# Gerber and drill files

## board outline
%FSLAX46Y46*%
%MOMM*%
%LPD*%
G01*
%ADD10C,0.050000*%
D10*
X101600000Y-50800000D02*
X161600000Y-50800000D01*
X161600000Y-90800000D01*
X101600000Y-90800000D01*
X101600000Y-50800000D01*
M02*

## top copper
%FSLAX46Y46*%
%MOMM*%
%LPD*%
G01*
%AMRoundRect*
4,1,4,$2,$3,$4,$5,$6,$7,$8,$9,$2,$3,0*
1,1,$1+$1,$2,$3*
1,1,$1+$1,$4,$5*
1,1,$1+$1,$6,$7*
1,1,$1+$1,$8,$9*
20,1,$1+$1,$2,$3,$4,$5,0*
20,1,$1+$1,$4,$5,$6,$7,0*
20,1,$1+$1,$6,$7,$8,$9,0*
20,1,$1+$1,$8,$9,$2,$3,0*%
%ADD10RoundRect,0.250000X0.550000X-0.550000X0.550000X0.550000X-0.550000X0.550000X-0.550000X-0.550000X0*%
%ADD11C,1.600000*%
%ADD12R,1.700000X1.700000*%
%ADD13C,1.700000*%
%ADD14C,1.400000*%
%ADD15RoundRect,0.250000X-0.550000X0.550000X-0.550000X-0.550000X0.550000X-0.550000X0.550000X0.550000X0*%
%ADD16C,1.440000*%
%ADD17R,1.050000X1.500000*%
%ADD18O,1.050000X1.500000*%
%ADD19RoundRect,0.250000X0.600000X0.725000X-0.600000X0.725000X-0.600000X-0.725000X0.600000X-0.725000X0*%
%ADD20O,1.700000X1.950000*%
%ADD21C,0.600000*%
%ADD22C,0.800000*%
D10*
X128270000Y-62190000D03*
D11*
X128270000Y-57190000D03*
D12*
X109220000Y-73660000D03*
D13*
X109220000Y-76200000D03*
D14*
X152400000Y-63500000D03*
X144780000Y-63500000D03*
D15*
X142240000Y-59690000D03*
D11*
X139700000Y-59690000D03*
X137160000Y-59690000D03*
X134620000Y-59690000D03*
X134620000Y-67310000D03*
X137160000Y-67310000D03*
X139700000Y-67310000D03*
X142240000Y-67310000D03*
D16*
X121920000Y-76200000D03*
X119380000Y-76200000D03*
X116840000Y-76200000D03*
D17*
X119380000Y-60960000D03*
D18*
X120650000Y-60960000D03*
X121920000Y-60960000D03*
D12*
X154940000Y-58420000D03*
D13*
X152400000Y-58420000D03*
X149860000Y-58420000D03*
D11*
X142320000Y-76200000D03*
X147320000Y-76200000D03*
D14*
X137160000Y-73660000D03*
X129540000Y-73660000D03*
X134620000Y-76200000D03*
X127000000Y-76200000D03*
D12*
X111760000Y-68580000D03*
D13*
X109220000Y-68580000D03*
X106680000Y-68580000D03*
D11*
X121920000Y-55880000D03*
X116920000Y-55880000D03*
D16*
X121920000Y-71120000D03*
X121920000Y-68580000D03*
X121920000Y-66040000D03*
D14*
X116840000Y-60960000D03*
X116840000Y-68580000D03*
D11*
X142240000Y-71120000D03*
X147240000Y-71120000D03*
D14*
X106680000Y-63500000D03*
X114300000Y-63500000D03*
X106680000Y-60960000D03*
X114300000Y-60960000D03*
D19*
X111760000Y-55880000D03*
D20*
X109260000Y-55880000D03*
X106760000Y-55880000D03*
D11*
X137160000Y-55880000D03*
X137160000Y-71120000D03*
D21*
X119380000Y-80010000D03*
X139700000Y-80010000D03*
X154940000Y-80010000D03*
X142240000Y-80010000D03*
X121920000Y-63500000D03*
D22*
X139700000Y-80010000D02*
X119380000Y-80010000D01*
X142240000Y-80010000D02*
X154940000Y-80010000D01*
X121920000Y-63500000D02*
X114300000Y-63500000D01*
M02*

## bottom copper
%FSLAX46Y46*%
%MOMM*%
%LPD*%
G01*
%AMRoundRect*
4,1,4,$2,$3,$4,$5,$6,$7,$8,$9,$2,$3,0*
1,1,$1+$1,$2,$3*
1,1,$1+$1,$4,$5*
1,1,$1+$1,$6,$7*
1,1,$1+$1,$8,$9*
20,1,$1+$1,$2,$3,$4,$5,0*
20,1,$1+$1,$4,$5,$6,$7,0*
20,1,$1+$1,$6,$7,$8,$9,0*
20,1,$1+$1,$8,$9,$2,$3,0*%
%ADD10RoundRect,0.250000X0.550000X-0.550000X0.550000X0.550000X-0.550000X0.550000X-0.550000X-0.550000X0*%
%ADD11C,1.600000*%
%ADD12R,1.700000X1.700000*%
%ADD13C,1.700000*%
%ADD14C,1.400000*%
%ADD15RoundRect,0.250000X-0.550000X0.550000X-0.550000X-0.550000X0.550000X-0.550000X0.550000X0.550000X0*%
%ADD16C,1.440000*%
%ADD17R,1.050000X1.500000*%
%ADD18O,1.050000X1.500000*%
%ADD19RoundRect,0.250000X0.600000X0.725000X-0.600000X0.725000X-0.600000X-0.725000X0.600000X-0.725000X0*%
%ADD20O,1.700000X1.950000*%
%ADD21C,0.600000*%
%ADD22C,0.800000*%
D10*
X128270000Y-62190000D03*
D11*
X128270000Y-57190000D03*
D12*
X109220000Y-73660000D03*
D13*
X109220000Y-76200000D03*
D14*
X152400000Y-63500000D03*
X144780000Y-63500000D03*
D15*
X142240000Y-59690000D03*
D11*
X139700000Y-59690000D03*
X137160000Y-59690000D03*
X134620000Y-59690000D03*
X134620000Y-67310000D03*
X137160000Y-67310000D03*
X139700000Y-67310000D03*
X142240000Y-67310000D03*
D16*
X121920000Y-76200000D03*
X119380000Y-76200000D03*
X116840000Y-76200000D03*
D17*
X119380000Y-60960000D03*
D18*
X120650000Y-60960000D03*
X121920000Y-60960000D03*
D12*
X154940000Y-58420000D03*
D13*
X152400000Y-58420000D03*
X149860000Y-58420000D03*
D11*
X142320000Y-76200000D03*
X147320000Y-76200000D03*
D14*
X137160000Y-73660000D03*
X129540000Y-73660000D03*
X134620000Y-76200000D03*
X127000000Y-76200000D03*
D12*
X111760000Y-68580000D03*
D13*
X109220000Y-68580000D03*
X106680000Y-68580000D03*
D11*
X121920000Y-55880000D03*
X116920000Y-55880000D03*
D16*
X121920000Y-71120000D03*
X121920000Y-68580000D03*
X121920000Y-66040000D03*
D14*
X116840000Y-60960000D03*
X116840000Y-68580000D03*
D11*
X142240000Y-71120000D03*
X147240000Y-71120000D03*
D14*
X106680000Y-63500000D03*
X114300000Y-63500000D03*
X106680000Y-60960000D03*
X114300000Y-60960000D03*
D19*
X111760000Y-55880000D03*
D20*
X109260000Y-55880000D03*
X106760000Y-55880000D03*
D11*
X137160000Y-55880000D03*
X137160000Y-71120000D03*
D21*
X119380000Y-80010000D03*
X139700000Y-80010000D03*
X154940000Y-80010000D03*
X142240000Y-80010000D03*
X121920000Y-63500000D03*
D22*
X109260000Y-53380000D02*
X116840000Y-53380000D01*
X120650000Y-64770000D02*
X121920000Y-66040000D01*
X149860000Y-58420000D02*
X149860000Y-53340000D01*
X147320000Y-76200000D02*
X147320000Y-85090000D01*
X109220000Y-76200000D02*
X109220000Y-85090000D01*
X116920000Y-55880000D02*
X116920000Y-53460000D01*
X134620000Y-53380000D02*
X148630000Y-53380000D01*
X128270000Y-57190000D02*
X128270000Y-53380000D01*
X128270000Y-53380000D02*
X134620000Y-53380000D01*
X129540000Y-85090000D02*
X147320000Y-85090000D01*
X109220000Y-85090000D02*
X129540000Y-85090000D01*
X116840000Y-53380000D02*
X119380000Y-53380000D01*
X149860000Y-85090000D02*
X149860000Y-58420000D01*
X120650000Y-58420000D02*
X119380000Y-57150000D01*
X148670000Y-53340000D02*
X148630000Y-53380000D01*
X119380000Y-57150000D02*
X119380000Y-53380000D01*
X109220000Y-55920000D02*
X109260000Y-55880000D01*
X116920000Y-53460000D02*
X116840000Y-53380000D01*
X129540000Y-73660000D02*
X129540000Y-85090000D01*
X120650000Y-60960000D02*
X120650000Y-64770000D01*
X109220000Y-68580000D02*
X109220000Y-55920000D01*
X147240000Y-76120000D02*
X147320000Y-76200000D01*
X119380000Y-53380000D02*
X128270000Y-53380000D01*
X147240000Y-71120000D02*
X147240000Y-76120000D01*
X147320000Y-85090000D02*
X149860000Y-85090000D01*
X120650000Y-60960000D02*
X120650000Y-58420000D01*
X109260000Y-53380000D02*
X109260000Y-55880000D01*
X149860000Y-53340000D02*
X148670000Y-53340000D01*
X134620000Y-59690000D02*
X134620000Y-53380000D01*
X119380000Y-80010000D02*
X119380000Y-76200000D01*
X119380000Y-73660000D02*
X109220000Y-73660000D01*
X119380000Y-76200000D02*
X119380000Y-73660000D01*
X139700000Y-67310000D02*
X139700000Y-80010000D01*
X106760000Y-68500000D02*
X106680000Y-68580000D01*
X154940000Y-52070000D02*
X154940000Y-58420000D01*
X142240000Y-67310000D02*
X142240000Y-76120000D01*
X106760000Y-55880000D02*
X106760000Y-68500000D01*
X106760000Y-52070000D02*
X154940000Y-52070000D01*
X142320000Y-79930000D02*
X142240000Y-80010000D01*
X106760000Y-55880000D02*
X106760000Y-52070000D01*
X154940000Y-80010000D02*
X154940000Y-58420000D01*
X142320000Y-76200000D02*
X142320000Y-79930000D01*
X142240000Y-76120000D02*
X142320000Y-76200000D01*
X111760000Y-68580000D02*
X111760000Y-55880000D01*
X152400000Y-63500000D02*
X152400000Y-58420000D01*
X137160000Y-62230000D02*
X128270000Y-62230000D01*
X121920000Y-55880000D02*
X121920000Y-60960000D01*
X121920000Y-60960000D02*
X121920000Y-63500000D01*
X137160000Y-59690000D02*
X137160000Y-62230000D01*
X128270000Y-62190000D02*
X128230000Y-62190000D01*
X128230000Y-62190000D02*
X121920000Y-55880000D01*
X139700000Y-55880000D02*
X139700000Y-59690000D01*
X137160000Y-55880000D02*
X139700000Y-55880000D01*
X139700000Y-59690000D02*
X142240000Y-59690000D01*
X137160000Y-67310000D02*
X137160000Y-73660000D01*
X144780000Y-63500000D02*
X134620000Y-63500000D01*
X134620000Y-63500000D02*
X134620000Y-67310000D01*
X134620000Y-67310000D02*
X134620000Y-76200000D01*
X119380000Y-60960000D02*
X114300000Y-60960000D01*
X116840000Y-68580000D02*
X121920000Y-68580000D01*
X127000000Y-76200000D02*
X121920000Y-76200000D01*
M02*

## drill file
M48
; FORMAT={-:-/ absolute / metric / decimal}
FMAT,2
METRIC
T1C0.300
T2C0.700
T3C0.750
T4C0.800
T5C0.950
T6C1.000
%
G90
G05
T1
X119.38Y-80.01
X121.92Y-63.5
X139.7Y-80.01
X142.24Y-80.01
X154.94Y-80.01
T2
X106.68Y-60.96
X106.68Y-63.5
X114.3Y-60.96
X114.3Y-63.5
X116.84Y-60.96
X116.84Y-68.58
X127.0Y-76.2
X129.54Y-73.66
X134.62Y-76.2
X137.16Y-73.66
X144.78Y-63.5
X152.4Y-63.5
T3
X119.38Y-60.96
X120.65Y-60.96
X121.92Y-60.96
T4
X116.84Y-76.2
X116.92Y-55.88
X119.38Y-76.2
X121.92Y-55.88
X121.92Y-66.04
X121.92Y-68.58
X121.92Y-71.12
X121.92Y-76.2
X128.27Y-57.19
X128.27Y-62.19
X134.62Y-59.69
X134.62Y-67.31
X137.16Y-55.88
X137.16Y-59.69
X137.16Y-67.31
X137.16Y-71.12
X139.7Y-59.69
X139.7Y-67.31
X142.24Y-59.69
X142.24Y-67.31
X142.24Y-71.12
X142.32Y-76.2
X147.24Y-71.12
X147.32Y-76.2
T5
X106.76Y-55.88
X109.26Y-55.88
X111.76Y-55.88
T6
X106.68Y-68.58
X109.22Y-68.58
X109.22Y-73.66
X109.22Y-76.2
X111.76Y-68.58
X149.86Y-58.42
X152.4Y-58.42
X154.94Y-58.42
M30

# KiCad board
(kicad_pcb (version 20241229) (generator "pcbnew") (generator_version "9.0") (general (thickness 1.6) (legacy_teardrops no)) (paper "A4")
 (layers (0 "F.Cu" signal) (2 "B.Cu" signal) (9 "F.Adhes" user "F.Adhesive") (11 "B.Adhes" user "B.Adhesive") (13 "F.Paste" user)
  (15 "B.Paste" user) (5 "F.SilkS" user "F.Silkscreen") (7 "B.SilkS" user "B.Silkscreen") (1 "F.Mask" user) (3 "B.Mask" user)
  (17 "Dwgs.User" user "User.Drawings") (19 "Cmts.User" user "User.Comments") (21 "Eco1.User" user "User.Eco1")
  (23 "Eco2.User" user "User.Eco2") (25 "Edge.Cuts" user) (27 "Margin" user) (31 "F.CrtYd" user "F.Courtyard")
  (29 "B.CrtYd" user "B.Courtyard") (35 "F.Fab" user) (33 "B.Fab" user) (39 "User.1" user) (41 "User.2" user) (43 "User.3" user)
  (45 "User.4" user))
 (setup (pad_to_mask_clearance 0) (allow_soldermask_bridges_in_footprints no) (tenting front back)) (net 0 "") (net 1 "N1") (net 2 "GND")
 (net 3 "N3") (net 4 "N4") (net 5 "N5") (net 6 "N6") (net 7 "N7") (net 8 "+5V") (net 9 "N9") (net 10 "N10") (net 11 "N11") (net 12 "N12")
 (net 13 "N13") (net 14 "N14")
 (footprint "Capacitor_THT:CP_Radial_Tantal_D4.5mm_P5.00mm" (layer "F.Cu") (at 128.27 62.19 90)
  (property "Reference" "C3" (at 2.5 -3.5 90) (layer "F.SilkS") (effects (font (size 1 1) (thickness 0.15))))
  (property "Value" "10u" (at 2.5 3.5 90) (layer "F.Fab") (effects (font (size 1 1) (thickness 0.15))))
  (pad "1" thru_hole roundrect (at 0 0 90) (size 1.6 1.6) (drill 0.8) (layers "*.Cu" "*.Mask") (remove_unused_layers no)
   (roundrect_rratio 0.15625) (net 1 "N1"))
  (pad "2" thru_hole circle (at 5 0 90) (size 1.6 1.6) (drill 0.8) (layers "*.Cu" "*.Mask") (remove_unused_layers no) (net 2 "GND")))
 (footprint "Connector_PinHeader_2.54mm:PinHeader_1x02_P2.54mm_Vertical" (layer "F.Cu") (at 109.22 73.66)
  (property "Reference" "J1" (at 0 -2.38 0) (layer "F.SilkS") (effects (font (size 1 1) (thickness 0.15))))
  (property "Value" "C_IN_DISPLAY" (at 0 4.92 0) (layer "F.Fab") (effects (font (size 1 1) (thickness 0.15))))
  (pad "1" thru_hole rect (at 0 0) (size 1.7 1.7) (drill 1) (layers "*.Cu" "*.Mask") (remove_unused_layers no) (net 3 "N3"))
  (pad "2" thru_hole circle (at 0 2.54) (size 1.7 1.7) (drill 1) (layers "*.Cu" "*.Mask") (remove_unused_layers no) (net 2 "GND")))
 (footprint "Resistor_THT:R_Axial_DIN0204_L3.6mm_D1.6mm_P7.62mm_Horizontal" (layer "F.Cu") (at 152.4 63.5 180)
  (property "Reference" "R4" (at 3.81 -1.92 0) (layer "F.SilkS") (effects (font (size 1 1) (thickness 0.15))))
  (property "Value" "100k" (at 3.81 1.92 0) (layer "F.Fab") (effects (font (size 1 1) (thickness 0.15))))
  (pad "1" thru_hole circle (at 0 0 180) (size 1.4 1.4) (drill 0.7) (layers "*.Cu" "*.Mask") (remove_unused_layers no) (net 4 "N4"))
  (pad "2" thru_hole circle (at 7.62 0 180) (size 1.4 1.4) (drill 0.7) (layers "*.Cu" "*.Mask") (remove_unused_layers no) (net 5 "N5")))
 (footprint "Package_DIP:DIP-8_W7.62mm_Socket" (layer "F.Cu") (at 142.24 59.69 -90)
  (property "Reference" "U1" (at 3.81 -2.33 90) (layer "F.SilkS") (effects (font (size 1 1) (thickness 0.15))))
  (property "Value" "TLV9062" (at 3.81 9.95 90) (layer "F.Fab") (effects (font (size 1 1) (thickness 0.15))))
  (pad "1" thru_hole roundrect (at 0 0 270) (size 1.6 1.6) (drill 0.8) (layers "*.Cu" "*.Mask") (remove_unused_layers no)
   (roundrect_rratio 0.15625) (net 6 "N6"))
  (pad "2" thru_hole circle (at 0 2.54 270) (size 1.6 1.6) (drill 0.8) (layers "*.Cu" "*.Mask") (remove_unused_layers no) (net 6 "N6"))
  (pad "3" thru_hole circle (at 0 5.08 270) (size 1.6 1.6) (drill 0.8) (layers "*.Cu" "*.Mask") (remove_unused_layers no) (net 1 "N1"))
  (pad "4" thru_hole circle (at 0 7.62 270) (size 1.6 1.6) (drill 0.8) (layers "*.Cu" "*.Mask") (remove_unused_layers no) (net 2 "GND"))
  (pad "5" thru_hole circle (at 7.62 7.62 270) (size 1.6 1.6) (drill 0.8) (layers "*.Cu" "*.Mask") (remove_unused_layers no) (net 5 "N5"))
  (pad "6" thru_hole circle (at 7.62 5.08 270) (size 1.6 1.6) (drill 0.8) (layers "*.Cu" "*.Mask") (remove_unused_layers no) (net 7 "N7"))
  (pad "7" thru_hole circle (at 7.62 2.54 270) (size 1.6 1.6) (drill 0.8) (layers "*.Cu" "*.Mask") (remove_unused_layers no) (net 3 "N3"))
  (pad "8" thru_hole circle (at 7.62 0 270) (size 1.6 1.6) (drill 0.8) (layers "*.Cu" "*.Mask") (remove_unused_layers no) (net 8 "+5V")))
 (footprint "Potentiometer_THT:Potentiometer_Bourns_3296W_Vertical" (layer "F.Cu") (at 121.92 76.2)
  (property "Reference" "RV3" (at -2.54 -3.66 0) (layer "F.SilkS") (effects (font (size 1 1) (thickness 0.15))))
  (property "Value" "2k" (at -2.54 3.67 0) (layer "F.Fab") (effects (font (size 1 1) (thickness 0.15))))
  (pad "1" thru_hole circle (at 0 0) (size 1.44 1.44) (drill 0.8) (layers "*.Cu" "*.Mask") (remove_unused_layers no) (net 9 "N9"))
  (pad "2" thru_hole circle (at -2.54 0) (size 1.44 1.44) (drill 0.8) (layers "*.Cu" "*.Mask") (remove_unused_layers no) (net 3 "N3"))
  (pad "3" thru_hole circle (at -5.08 0) (size 1.44 1.44) (drill 0.8) (layers "*.Cu" "*.Mask") (remove_unused_layers no) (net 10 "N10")))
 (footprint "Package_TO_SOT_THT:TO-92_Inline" (layer "F.Cu") (at 119.38 60.96)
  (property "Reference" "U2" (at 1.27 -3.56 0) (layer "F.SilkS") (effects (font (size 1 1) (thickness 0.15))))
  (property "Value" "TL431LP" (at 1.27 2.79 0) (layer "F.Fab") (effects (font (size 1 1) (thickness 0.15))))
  (pad "1" thru_hole rect (at 0 0) (size 1.05 1.5) (drill 0.75) (layers "*.Cu" "*.Mask") (remove_unused_layers no) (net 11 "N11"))
  (pad "2" thru_hole oval (at 1.27 0) (size 1.05 1.5) (drill 0.75) (layers "*.Cu" "*.Mask") (remove_unused_layers no) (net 2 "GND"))
  (pad "3" thru_hole oval (at 2.54 0) (size 1.05 1.5) (drill 0.75) (layers "*.Cu" "*.Mask") (remove_unused_layers no) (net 1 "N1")))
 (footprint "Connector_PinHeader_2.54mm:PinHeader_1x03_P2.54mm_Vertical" (layer "F.Cu") (at 154.94 58.42 -90)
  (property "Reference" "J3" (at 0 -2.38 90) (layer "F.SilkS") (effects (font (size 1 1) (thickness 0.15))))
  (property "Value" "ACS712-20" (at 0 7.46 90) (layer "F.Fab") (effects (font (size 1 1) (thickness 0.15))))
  (pad "1" thru_hole rect (at 0 0 270) (size 1.7 1.7) (drill 1) (layers "*.Cu" "*.Mask") (remove_unused_layers no) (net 8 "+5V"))
  (pad "2" thru_hole circle (at 0 2.54 270) (size 1.7 1.7) (drill 1) (layers "*.Cu" "*.Mask") (remove_unused_layers no) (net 4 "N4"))
  (pad "3" thru_hole circle (at 0 5.08 270) (size 1.7 1.7) (drill 1) (layers "*.Cu" "*.Mask") (remove_unused_layers no) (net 2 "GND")))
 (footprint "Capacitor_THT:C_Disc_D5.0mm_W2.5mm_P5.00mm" (layer "F.Cu") (at 142.32 76.2)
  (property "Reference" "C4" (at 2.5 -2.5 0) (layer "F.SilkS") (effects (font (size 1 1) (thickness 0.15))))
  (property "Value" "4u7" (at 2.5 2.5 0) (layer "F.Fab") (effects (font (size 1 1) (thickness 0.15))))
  (pad "1" thru_hole circle (at 0 0) (size 1.6 1.6) (drill 0.8) (layers "*.Cu" "*.Mask") (remove_unused_layers no) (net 8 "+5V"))
  (pad "2" thru_hole circle (at 5 0) (size 1.6 1.6) (drill 0.8) (layers "*.Cu" "*.Mask") (remove_unused_layers no) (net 2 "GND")))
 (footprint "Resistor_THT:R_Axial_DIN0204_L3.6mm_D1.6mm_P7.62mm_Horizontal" (layer "F.Cu") (at 137.16 73.66 180)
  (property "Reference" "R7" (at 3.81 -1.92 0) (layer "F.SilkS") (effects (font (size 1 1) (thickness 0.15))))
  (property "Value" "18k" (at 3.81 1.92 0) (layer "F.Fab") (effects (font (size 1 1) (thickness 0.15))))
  (pad "1" thru_hole circle (at 0 0 180) (size 1.4 1.4) (drill 0.7) (layers "*.Cu" "*.Mask") (remove_unused_layers no) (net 7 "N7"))
  (pad "2" thru_hole circle (at 7.62 0 180) (size 1.4 1.4) (drill 0.7) (layers "*.Cu" "*.Mask") (remove_unused_layers no) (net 2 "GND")))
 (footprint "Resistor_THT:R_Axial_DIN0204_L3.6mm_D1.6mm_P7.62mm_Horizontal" (layer "F.Cu") (at 134.62 76.2 180)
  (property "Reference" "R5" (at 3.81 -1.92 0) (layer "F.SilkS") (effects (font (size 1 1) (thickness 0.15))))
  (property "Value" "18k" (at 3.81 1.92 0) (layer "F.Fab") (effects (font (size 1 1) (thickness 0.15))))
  (pad "1" thru_hole circle (at 0 0 180) (size 1.4 1.4) (drill 0.7) (layers "*.Cu" "*.Mask") (remove_unused_layers no) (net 5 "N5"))
  (pad "2" thru_hole circle (at 7.62 0 180) (size 1.4 1.4) (drill 0.7) (layers "*.Cu" "*.Mask") (remove_unused_layers no) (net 9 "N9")))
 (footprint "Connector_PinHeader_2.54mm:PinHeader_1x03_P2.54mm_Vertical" (layer "F.Cu") (at 111.76 68.58 -90)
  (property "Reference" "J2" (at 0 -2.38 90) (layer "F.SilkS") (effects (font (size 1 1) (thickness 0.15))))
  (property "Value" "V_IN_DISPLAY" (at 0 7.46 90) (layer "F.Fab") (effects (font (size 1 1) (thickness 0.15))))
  (pad "1" thru_hole rect (at 0 0 270) (size 1.7 1.7) (drill 1) (layers "*.Cu" "*.Mask") (remove_unused_layers no) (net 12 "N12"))
  (pad "2" thru_hole circle (at 0 2.54 270) (size 1.7 1.7) (drill 1) (layers "*.Cu" "*.Mask") (remove_unused_layers no) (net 2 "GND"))
  (pad "3" thru_hole circle (at 0 5.08 270) (size 1.7 1.7) (drill 1) (layers "*.Cu" "*.Mask") (remove_unused_layers no) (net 8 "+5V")))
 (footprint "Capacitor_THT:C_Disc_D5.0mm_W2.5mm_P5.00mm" (layer "F.Cu") (at 121.92 55.88 180)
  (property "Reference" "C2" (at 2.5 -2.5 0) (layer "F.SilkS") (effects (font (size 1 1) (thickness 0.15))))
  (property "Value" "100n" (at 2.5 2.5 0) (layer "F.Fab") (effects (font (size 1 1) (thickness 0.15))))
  (pad "1" thru_hole circle (at 0 0 180) (size 1.6 1.6) (drill 0.8) (layers "*.Cu" "*.Mask") (remove_unused_layers no) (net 1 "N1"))
  (pad "2" thru_hole circle (at 5 0 180) (size 1.6 1.6) (drill 0.8) (layers "*.Cu" "*.Mask") (remove_unused_layers no) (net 2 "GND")))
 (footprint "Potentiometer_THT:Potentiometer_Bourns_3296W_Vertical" (layer "F.Cu") (at 121.92 71.12 -90)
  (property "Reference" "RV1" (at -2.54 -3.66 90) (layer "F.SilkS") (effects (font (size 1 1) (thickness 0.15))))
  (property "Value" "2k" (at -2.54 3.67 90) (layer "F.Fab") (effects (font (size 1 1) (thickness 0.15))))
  (pad "1" thru_hole circle (at 0 0 270) (size 1.44 1.44) (drill 0.8) (layers "*.Cu" "*.Mask") (remove_unused_layers no) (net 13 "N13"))
  (pad "2" thru_hole circle (at -2.54 0 270) (size 1.44 1.44) (drill 0.8) (layers "*.Cu" "*.Mask") (remove_unused_layers no) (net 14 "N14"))
  (pad "3" thru_hole circle (at -5.08 0 270) (size 1.44 1.44) (drill 0.8) (layers "*.Cu" "*.Mask") (remove_unused_layers no) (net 2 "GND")))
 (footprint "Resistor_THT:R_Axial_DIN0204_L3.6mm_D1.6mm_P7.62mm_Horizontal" (layer "F.Cu") (at 116.84 60.96 -90)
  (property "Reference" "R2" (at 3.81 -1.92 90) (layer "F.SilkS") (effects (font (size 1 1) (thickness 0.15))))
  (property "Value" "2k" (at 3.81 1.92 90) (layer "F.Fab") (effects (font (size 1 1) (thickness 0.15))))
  (pad "1" thru_hole circle (at 0 0 270) (size 1.4 1.4) (drill 0.7) (layers "*.Cu" "*.Mask") (remove_unused_layers no) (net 11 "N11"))
  (pad "2" thru_hole circle (at 7.62 0 270) (size 1.4 1.4) (drill 0.7) (layers "*.Cu" "*.Mask") (remove_unused_layers no) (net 14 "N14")))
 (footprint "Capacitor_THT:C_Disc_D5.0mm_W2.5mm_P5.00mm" (layer "F.Cu") (at 142.24 71.12)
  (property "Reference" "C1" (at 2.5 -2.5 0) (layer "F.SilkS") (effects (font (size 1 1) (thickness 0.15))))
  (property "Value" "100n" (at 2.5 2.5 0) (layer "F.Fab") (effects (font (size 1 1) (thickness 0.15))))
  (pad "1" thru_hole circle (at 0 0) (size 1.6 1.6) (drill 0.8) (layers "*.Cu" "*.Mask") (remove_unused_layers no) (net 8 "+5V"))
  (pad "2" thru_hole circle (at 5 0) (size 1.6 1.6) (drill 0.8) (layers "*.Cu" "*.Mask") (remove_unused_layers no) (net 2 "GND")))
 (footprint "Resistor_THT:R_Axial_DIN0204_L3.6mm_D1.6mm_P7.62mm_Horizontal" (layer "F.Cu") (at 106.68 63.5)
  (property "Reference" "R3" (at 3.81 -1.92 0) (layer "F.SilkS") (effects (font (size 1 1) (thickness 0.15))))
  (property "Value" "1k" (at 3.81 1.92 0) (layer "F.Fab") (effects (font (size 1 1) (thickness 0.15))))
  (pad "1" thru_hole circle (at 0 0) (size 1.4 1.4) (drill 0.7) (layers "*.Cu" "*.Mask") (remove_unused_layers no) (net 8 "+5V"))
  (pad "2" thru_hole circle (at 7.62 0) (size 1.4 1.4) (drill 0.7) (layers "*.Cu" "*.Mask") (remove_unused_layers no) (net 1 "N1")))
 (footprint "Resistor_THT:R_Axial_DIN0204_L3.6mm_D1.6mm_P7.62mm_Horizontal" (layer "F.Cu") (at 106.68 60.96)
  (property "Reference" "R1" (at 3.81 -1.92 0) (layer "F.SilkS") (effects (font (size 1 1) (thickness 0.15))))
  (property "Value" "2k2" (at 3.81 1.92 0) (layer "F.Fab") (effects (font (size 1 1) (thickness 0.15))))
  (pad "1" thru_hole circle (at 0 0) (size 1.4 1.4) (drill 0.7) (layers "*.Cu" "*.Mask") (remove_unused_layers no) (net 8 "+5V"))
  (pad "2" thru_hole circle (at 7.62 0) (size 1.4 1.4) (drill 0.7) (layers "*.Cu" "*.Mask") (remove_unused_layers no) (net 11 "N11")))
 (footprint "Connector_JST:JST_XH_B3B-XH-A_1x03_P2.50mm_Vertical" (layer "F.Cu") (at 111.76 55.88 180)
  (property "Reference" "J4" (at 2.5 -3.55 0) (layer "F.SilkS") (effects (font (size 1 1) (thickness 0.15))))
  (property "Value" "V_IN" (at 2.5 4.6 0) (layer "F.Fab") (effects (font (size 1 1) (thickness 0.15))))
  (pad "1" thru_hole roundrect (at 0 0 180) (size 1.7 1.95) (drill 0.95) (layers "*.Cu" "*.Mask") (remove_unused_layers no)
   (roundrect_rratio 0.147059) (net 12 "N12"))
  (pad "2" thru_hole oval (at 2.5 0 180) (size 1.7 1.95) (drill 0.95) (layers "*.Cu" "*.Mask") (remove_unused_layers no) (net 2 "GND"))
  (pad "3" thru_hole oval (at 5 0 180) (size 1.7 1.95) (drill 0.95) (layers "*.Cu" "*.Mask") (remove_unused_layers no) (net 8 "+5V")))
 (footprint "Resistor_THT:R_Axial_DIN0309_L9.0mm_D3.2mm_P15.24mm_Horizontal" (layer "B.Cu") (at 137.16 55.88 -90)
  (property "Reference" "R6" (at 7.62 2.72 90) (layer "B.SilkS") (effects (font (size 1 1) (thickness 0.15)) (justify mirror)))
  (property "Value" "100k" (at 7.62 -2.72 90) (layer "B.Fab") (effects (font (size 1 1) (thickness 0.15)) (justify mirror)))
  (pad "1" thru_hole circle (at 0 0 270) (size 1.6 1.6) (drill 0.8) (layers "*.Cu" "*.Mask") (remove_unused_layers no) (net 6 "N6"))
  (pad "2" thru_hole circle (at 15.24 0 270) (size 1.6 1.6) (drill 0.8) (layers "*.Cu" "*.Mask") (remove_unused_layers no) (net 7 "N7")))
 (gr_rect (start 101.6 50.8) (end 161.6 90.8) (stroke (width 0.05) (type solid)) (fill no) (layer "Edge.Cuts"))
 (segment (start 109.26 53.38) (end 116.84 53.38) (width 0.8) (layer "B.Cu") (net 2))
 (segment (start 120.65 64.77) (end 121.92 66.04) (width 0.8) (layer "B.Cu") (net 2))
 (segment (start 149.86 58.42) (end 149.86 53.34) (width 0.8) (layer "B.Cu") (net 2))
 (segment (start 147.32 76.2) (end 147.32 85.09) (width 0.8) (layer "B.Cu") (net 2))
 (segment (start 109.22 76.2) (end 109.22 85.09) (width 0.8) (layer "B.Cu") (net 2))
 (segment (start 116.92 55.88) (end 116.92 53.46) (width 0.8) (layer "B.Cu") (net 2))
 (segment (start 134.62 53.38) (end 148.63 53.38) (width 0.8) (layer "B.Cu") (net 2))
 (segment (start 128.27 57.19) (end 128.27 53.38) (width 0.8) (layer "B.Cu") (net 2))
 (segment (start 128.27 53.38) (end 134.62 53.38) (width 0.8) (layer "B.Cu") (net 2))
 (segment (start 129.54 85.09) (end 147.32 85.09) (width 0.8) (layer "B.Cu") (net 2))
 (segment (start 109.22 85.09) (end 129.54 85.09) (width 0.8) (layer "B.Cu") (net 2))
 (segment (start 116.84 53.38) (end 119.38 53.38) (width 0.8) (layer "B.Cu") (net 2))
 (segment (start 149.86 85.09) (end 149.86 58.42) (width 0.8) (layer "B.Cu") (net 2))
 (segment (start 120.65 58.42) (end 119.38 57.15) (width 0.8) (layer "B.Cu") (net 2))
 (segment (start 148.67 53.34) (end 148.63 53.38) (width 0.8) (layer "B.Cu") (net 2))
 (segment (start 119.38 57.15) (end 119.38 53.38) (width 0.8) (layer "B.Cu") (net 2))
 (segment (start 109.22 55.92) (end 109.26 55.88) (width 0.8) (layer "B.Cu") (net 2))
 (segment (start 116.92 53.46) (end 116.84 53.38) (width 0.8) (layer "B.Cu") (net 2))
 (segment (start 129.54 73.66) (end 129.54 85.09) (width 0.8) (layer "B.Cu") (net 2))
 (segment (start 120.65 60.96) (end 120.65 64.77) (width 0.8) (layer "B.Cu") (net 2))
 (segment (start 109.22 68.58) (end 109.22 55.92) (width 0.8) (layer "B.Cu") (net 2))
 (segment (start 147.24 76.12) (end 147.32 76.2) (width 0.8) (layer "B.Cu") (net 2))
 (segment (start 119.38 53.38) (end 128.27 53.38) (width 0.8) (layer "B.Cu") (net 2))
 (segment (start 147.24 71.12) (end 147.24 76.12) (width 0.8) (layer "B.Cu") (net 2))
 (segment (start 147.32 85.09) (end 149.86 85.09) (width 0.8) (layer "B.Cu") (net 2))
 (segment (start 120.65 60.96) (end 120.65 58.42) (width 0.8) (layer "B.Cu") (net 2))
 (segment (start 109.26 53.38) (end 109.26 55.88) (width 0.8) (layer "B.Cu") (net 2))
 (segment (start 149.86 53.34) (end 148.67 53.34) (width 0.8) (layer "B.Cu") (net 2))
 (segment (start 134.62 59.69) (end 134.62 53.38) (width 0.8) (layer "B.Cu") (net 2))
 (segment (start 139.7 80.01) (end 119.38 80.01) (width 0.8) (layer "F.Cu") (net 3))
 (via (at 119.38 80.01) (size 0.6) (drill 0.3) (layers "F.Cu" "B.Cu") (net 3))
 (via (at 139.7 80.01) (size 0.6) (drill 0.3) (layers "F.Cu" "B.Cu") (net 3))
 (segment (start 119.38 80.01) (end 119.38 76.2) (width 0.8) (layer "B.Cu") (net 3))
 (segment (start 119.38 73.66) (end 109.22 73.66) (width 0.8) (layer "B.Cu") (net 3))
 (segment (start 119.38 76.2) (end 119.38 73.66) (width 0.8) (layer "B.Cu") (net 3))
 (segment (start 139.7 67.31) (end 139.7 80.01) (width 0.8) (layer "B.Cu") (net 3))
 (segment (start 142.24 80.01) (end 154.94 80.01) (width 0.8) (layer "F.Cu") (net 8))
 (via (at 154.94 80.01) (size 0.6) (drill 0.3) (layers "F.Cu" "B.Cu") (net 8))
 (via (at 142.24 80.01) (size 0.6) (drill 0.3) (layers "F.Cu" "B.Cu") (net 8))
 (segment (start 106.76 68.5) (end 106.68 68.58) (width 0.8) (layer "B.Cu") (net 8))
 (segment (start 154.94 52.07) (end 154.94 58.42) (width 0.8) (layer "B.Cu") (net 8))
 (segment (start 142.24 67.31) (end 142.24 76.12) (width 0.8) (layer "B.Cu") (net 8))
 (segment (start 106.76 55.88) (end 106.76 68.5) (width 0.8) (layer "B.Cu") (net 8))
 (segment (start 106.76 52.07) (end 154.94 52.07) (width 0.8) (layer "B.Cu") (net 8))
 (segment (start 142.32 79.93) (end 142.24 80.01) (width 0.8) (layer "B.Cu") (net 8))
 (segment (start 106.76 55.88) (end 106.76 52.07) (width 0.8) (layer "B.Cu") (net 8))
 (segment (start 154.94 80.01) (end 154.94 58.42) (width 0.8) (layer "B.Cu") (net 8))
 (segment (start 142.32 76.2) (end 142.32 79.93) (width 0.8) (layer "B.Cu") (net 8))
 (segment (start 142.24 76.12) (end 142.32 76.2) (width 0.8) (layer "B.Cu") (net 8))
 (segment (start 111.76 68.58) (end 111.76 55.88) (width 0.8) (layer "B.Cu") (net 12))
 (segment (start 152.4 63.5) (end 152.4 58.42) (width 0.8) (layer "B.Cu") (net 4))
 (segment (start 121.92 63.5) (end 114.3 63.5) (width 0.8) (layer "F.Cu") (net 1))
 (via (at 121.92 63.5) (size 0.6) (drill 0.3) (layers "F.Cu" "B.Cu") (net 1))
 (segment (start 137.16 62.23) (end 128.27 62.23) (width 0.8) (layer "B.Cu") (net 1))
 (segment (start 121.92 55.88) (end 121.92 60.96) (width 0.8) (layer "B.Cu") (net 1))
 (segment (start 121.92 60.96) (end 121.92 63.5) (width 0.8) (layer "B.Cu") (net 1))
 (segment (start 137.16 59.69) (end 137.16 62.23) (width 0.8) (layer "B.Cu") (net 1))
 (segment (start 128.27 62.19) (end 128.23 62.19) (width 0.8) (layer "B.Cu") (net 1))
 (segment (start 128.23 62.19) (end 121.92 55.88) (width 0.8) (layer "B.Cu") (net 1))
 (segment (start 139.7 55.88) (end 139.7 59.69) (width 0.8) (layer "B.Cu") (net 6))
 (segment (start 137.16 55.88) (end 139.7 55.88) (width 0.8) (layer "B.Cu") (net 6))
 (segment (start 139.7 59.69) (end 142.24 59.69) (width 0.8) (layer "B.Cu") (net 6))
 (segment (start 137.16 67.31) (end 137.16 73.66) (width 0.8) (layer "B.Cu") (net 7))
 (segment (start 144.78 63.5) (end 134.62 63.5) (width 0.8) (layer "B.Cu") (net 5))
 (segment (start 134.62 63.5) (end 134.62 67.31) (width 0.8) (layer "B.Cu") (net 5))
 (segment (start 134.62 67.31) (end 134.62 76.2) (width 0.8) (layer "B.Cu") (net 5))
 (segment (start 119.38 60.96) (end 114.3 60.96) (width 0.8) (layer "B.Cu") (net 11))
 (segment (start 116.84 68.58) (end 121.92 68.58) (width 0.8) (layer "B.Cu") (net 14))
 (segment (start 127 76.2) (end 121.92 76.2) (width 0.8) (layer "B.Cu") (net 9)))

